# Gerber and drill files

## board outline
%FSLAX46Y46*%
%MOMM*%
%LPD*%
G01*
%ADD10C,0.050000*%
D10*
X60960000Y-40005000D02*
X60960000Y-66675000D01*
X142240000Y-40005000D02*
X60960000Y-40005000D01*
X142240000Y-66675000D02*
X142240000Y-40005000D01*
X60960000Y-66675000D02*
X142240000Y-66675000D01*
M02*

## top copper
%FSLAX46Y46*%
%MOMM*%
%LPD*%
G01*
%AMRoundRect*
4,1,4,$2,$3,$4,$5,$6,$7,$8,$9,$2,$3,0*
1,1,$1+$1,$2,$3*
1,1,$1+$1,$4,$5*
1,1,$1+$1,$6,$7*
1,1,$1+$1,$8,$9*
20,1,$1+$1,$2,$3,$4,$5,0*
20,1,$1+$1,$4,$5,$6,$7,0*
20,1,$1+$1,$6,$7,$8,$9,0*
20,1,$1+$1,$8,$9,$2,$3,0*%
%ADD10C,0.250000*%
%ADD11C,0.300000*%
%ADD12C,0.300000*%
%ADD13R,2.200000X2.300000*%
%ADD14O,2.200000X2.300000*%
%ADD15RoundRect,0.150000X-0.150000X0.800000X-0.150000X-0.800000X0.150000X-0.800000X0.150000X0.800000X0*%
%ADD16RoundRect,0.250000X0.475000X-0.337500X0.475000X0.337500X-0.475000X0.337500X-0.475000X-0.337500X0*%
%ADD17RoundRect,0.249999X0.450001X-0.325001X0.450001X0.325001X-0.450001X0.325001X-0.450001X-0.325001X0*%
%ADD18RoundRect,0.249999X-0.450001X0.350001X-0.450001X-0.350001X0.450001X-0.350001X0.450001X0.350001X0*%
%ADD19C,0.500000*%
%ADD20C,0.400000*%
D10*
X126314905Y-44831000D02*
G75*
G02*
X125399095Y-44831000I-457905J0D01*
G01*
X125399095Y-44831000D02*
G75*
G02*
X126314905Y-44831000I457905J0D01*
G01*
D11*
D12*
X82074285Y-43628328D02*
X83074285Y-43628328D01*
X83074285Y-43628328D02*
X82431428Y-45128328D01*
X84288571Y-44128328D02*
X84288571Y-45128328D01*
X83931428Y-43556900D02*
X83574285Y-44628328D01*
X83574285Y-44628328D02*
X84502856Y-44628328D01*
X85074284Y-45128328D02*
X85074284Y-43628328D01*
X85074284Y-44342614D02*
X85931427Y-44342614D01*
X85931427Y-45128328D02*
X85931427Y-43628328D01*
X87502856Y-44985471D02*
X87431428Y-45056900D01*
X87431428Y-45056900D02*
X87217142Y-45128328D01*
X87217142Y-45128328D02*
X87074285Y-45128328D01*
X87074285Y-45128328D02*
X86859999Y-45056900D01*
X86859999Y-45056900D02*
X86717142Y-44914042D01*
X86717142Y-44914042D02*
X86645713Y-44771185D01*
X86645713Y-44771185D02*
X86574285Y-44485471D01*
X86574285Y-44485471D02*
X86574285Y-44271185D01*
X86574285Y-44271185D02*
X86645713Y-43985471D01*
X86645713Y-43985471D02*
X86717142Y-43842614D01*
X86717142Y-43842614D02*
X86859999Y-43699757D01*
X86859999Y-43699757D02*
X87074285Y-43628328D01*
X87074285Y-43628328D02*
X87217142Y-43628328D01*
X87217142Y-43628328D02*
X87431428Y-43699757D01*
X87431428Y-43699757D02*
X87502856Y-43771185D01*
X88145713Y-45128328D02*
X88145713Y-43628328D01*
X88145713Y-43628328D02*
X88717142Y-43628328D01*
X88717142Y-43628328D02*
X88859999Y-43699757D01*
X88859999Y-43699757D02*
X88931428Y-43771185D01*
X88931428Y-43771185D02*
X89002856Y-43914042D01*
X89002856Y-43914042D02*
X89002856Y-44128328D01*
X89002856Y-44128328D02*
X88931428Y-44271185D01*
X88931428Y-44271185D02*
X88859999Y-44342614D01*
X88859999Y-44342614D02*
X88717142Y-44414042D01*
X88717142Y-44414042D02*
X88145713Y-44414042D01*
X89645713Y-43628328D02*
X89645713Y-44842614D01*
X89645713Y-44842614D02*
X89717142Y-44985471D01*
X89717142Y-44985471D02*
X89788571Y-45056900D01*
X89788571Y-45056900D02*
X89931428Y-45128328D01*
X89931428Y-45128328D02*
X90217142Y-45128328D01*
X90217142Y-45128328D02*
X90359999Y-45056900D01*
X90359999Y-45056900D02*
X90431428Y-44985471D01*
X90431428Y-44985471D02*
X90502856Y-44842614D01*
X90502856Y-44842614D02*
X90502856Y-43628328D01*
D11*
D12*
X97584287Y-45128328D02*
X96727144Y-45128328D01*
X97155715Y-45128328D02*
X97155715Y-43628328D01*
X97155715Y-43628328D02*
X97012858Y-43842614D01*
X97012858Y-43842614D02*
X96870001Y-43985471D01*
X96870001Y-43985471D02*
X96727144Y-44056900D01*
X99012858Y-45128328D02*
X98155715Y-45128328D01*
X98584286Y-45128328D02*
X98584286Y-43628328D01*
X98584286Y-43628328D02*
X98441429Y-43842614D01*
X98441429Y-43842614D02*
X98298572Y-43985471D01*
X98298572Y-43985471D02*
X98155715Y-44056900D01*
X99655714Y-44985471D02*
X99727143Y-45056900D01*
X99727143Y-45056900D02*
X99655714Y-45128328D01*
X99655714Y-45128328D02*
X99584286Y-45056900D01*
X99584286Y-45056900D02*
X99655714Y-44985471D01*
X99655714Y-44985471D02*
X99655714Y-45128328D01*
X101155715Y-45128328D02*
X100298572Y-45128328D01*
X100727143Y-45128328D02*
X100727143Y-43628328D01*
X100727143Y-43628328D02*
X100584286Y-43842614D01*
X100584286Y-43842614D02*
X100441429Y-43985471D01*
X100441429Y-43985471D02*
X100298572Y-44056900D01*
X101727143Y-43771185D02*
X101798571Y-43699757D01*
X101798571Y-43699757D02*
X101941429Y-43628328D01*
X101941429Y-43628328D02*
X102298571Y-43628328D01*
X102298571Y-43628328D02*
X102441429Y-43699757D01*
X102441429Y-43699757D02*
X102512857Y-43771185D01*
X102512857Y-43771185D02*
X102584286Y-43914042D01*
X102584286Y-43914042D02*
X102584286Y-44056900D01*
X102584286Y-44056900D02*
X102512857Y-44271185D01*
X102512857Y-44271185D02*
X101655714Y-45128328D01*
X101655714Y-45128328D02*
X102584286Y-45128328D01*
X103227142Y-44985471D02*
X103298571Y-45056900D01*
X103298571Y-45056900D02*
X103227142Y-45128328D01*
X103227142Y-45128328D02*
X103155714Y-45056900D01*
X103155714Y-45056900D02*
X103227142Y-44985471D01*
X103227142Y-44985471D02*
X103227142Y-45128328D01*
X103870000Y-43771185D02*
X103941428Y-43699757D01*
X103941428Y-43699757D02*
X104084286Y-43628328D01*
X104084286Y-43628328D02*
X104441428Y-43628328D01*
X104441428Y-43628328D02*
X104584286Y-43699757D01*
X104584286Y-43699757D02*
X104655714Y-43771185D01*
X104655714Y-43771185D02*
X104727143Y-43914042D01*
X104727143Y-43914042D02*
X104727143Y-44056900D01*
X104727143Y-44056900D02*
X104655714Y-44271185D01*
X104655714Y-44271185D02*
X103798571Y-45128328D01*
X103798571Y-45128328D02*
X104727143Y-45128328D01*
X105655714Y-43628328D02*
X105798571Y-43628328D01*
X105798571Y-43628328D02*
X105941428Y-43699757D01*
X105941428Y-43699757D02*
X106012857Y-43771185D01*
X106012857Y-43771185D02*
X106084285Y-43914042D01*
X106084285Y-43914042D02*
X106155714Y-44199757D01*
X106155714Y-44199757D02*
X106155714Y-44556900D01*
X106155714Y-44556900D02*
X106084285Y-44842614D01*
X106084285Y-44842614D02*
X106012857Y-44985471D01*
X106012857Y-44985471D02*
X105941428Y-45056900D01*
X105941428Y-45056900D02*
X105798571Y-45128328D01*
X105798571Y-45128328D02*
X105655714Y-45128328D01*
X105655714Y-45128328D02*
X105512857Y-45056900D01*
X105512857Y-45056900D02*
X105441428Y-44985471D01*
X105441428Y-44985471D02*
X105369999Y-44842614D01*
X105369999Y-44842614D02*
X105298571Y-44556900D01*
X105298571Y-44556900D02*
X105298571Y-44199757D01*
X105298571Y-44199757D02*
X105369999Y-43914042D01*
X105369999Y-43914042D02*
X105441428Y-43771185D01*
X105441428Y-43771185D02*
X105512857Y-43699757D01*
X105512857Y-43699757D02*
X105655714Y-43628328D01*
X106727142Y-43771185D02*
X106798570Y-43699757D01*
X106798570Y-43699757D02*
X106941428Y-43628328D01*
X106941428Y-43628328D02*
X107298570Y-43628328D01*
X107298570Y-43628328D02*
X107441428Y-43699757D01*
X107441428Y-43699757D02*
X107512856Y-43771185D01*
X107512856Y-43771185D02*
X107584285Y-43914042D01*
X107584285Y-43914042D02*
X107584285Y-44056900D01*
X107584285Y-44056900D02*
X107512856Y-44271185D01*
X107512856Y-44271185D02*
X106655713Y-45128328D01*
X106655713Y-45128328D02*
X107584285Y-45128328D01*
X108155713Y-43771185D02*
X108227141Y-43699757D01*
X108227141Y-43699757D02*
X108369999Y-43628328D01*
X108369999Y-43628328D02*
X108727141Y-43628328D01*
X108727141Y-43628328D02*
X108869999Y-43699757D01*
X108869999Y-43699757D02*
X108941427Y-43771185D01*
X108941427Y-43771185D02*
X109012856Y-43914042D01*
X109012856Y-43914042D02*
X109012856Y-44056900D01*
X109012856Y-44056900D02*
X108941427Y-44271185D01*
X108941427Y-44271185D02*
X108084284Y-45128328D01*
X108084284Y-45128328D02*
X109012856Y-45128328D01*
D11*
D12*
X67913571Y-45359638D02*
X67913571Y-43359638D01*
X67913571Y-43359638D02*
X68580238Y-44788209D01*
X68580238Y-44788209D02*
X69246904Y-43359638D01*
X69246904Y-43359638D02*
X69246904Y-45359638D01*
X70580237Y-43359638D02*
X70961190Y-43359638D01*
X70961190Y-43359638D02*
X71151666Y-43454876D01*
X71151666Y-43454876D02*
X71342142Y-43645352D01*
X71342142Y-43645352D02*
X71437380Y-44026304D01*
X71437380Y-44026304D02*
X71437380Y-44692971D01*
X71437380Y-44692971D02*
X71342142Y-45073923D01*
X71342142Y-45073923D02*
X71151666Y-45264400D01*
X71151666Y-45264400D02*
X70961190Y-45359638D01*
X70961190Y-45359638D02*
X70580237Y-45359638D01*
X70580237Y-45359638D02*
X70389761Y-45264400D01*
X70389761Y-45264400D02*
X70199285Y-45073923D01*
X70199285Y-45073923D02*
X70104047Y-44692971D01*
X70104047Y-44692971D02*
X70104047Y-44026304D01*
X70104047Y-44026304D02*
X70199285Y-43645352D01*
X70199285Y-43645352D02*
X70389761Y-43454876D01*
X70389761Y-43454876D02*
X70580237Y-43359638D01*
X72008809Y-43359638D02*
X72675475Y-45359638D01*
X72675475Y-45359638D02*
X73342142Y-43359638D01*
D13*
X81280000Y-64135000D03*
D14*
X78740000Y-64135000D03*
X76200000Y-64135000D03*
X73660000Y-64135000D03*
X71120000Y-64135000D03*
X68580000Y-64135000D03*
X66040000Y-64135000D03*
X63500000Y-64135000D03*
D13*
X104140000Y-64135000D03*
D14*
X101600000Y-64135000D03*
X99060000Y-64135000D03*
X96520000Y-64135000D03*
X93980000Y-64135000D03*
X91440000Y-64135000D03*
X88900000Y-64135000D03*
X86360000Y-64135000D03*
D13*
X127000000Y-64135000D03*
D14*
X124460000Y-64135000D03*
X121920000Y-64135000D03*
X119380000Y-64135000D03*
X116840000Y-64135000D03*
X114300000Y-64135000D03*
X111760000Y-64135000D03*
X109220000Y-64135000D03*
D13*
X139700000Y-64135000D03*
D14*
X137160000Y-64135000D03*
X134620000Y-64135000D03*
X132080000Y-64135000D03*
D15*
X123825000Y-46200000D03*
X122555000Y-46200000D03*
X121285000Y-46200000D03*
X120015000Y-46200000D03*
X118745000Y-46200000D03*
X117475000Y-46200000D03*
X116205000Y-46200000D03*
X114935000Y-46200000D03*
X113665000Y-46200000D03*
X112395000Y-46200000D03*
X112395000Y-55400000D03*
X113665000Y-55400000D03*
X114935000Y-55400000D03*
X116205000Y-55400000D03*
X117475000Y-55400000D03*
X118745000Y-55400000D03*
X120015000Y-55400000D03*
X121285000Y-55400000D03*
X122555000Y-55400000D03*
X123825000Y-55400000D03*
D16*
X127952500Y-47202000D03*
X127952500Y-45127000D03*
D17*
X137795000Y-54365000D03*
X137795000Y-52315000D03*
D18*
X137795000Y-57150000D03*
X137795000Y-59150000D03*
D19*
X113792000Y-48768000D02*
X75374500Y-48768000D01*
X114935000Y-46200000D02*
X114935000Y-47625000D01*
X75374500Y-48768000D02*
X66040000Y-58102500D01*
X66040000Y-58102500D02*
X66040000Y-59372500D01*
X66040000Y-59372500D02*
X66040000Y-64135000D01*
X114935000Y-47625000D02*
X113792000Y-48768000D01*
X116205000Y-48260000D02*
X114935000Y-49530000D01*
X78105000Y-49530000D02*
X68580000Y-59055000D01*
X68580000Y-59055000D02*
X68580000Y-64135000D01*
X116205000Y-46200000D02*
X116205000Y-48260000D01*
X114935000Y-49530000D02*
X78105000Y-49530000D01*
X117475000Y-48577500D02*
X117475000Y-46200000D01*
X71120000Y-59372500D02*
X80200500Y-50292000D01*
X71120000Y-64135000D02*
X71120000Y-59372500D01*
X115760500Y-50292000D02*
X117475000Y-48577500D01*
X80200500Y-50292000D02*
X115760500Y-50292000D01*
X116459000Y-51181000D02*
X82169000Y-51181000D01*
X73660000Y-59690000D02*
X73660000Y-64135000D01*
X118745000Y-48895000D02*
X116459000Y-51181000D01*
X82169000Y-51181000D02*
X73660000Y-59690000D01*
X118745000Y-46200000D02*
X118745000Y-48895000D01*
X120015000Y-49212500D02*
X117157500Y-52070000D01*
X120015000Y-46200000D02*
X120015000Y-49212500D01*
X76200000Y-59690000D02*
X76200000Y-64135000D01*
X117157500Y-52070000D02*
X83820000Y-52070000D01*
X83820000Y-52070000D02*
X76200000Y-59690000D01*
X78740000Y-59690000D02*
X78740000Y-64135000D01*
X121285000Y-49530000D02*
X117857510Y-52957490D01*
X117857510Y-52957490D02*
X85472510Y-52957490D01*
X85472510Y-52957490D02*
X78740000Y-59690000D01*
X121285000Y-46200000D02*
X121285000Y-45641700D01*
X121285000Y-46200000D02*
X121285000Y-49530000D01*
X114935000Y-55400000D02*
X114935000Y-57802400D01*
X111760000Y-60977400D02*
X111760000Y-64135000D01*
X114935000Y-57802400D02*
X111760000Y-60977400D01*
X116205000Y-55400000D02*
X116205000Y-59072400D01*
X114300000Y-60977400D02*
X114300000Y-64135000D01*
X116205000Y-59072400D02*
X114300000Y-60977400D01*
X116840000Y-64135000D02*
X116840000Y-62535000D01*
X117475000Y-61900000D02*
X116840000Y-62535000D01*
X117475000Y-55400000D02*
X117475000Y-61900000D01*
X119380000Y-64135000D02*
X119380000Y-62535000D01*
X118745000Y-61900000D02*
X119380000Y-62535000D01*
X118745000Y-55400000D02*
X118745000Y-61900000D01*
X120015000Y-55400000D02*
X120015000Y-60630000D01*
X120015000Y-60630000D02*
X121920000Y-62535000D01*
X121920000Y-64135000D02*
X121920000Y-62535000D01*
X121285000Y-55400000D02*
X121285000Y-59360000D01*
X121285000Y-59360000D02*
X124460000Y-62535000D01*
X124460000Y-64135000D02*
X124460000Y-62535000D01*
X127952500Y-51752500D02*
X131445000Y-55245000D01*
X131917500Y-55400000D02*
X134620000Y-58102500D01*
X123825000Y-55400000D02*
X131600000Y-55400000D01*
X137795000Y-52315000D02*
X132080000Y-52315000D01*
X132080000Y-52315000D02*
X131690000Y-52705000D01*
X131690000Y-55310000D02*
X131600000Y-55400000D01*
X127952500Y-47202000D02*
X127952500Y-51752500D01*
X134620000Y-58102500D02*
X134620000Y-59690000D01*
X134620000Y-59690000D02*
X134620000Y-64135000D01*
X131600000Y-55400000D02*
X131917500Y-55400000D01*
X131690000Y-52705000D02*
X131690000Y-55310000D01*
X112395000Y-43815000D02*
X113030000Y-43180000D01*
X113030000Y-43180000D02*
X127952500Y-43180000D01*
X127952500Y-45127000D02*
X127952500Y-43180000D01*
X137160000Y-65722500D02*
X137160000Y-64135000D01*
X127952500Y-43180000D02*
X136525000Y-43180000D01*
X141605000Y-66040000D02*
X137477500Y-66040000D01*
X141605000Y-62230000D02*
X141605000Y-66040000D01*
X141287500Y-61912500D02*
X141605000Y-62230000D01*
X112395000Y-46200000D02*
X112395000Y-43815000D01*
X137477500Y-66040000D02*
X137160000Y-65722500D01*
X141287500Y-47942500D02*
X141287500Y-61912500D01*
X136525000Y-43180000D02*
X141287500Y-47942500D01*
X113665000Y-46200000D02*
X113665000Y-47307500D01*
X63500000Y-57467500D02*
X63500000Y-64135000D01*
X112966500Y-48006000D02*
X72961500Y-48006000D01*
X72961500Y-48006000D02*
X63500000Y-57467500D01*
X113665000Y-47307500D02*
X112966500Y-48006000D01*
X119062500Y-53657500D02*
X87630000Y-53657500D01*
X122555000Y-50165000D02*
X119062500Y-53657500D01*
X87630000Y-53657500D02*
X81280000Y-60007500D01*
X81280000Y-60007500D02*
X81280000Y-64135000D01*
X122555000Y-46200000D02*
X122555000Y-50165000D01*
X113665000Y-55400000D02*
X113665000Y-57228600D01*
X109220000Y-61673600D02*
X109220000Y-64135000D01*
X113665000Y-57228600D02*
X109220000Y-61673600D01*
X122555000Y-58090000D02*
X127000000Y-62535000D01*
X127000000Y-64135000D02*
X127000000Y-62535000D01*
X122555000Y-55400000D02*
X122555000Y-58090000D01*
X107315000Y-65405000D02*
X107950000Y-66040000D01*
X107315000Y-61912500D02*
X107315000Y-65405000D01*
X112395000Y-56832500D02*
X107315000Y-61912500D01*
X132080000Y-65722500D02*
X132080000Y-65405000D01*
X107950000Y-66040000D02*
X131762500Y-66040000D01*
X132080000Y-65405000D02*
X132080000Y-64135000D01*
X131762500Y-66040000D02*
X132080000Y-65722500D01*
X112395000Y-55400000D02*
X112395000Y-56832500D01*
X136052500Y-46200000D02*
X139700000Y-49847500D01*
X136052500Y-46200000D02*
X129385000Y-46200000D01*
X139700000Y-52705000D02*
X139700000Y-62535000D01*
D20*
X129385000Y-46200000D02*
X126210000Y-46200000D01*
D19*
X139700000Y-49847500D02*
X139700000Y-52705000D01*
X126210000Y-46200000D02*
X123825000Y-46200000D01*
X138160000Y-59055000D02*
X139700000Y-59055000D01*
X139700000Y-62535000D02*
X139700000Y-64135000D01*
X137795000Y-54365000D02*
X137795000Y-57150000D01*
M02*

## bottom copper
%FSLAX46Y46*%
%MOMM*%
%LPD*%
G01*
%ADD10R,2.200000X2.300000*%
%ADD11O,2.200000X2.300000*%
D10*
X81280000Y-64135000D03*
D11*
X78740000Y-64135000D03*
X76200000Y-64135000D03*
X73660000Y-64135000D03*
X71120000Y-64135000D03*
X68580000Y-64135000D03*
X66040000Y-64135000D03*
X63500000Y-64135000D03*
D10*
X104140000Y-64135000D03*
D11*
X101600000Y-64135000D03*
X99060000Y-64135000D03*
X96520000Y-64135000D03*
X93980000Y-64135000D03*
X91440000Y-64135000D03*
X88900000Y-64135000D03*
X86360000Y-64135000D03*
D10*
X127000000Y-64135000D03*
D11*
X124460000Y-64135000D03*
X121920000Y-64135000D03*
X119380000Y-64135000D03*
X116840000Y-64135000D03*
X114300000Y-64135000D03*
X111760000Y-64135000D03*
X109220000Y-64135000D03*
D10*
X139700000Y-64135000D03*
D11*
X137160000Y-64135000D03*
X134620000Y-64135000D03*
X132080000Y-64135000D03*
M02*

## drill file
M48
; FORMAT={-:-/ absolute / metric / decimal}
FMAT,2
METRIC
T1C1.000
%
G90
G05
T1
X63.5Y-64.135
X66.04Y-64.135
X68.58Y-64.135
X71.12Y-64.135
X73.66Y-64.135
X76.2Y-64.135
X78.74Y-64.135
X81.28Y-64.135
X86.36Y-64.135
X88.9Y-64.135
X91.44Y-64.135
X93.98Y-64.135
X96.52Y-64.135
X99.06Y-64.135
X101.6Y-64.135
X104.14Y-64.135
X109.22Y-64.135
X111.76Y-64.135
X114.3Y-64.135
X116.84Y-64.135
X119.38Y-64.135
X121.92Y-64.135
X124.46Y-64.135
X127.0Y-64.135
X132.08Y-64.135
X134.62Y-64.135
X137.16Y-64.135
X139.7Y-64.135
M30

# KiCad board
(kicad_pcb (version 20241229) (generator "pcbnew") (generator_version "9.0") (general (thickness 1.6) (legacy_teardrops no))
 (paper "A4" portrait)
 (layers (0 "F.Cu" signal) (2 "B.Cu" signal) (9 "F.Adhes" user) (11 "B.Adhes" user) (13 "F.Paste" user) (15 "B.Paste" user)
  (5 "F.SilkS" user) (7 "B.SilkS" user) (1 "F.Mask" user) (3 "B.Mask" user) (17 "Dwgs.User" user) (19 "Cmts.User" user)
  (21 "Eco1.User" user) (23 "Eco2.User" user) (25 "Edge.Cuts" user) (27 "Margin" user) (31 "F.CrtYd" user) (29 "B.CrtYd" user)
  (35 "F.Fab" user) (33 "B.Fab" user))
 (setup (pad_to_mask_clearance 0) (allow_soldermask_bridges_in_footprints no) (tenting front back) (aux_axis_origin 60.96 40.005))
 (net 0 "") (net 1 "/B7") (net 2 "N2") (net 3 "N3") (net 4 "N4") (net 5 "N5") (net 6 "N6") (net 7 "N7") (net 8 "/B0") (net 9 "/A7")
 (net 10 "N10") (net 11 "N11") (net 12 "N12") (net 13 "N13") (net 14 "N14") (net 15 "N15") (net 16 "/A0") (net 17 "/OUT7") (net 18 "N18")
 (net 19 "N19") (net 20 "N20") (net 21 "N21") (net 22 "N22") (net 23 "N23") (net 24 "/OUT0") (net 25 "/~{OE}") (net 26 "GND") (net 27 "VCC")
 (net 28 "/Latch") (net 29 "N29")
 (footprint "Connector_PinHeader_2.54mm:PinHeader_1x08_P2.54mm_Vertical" (layer "F.Cu") (at 81.28 64.135 -90)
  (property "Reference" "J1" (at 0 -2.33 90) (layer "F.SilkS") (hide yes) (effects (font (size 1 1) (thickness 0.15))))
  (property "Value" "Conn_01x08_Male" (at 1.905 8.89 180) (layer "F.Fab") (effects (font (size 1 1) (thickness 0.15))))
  (pad "1" thru_hole rect (at 0 0 270) (size 2.3 2.2) (drill 1) (layers "*.Cu" "*.Mask") (remove_unused_layers no) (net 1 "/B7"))
  (pad "2" thru_hole oval (at 0 2.54 270) (size 2.3 2.2) (drill 1) (layers "*.Cu" "*.Mask") (remove_unused_layers no) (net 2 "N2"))
  (pad "3" thru_hole oval (at 0 5.08 270) (size 2.3 2.2) (drill 1) (layers "*.Cu" "*.Mask") (remove_unused_layers no) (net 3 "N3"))
  (pad "4" thru_hole oval (at 0 7.62 270) (size 2.3 2.2) (drill 1) (layers "*.Cu" "*.Mask") (remove_unused_layers no) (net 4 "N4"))
  (pad "5" thru_hole oval (at 0 10.16 270) (size 2.3 2.2) (drill 1) (layers "*.Cu" "*.Mask") (remove_unused_layers no) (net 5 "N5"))
  (pad "6" thru_hole oval (at 0 12.7 270) (size 2.3 2.2) (drill 1) (layers "*.Cu" "*.Mask") (remove_unused_layers no) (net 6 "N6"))
  (pad "7" thru_hole oval (at 0 15.24 270) (size 2.3 2.2) (drill 1) (layers "*.Cu" "*.Mask") (remove_unused_layers no) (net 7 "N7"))
  (pad "8" thru_hole oval (at 0 17.78 270) (size 2.3 2.2) (drill 1) (layers "*.Cu" "*.Mask") (remove_unused_layers no) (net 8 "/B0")))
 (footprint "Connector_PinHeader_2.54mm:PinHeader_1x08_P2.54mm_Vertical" (layer "F.Cu") (at 104.14 64.135 -90)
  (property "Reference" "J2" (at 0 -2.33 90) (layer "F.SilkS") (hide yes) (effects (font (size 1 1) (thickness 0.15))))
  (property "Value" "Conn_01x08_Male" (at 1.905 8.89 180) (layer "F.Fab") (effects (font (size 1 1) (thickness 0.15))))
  (pad "1" thru_hole rect (at 0 0 270) (size 2.3 2.2) (drill 1) (layers "*.Cu" "*.Mask") (remove_unused_layers no) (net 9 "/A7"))
  (pad "2" thru_hole oval (at 0 2.54 270) (size 2.3 2.2) (drill 1) (layers "*.Cu" "*.Mask") (remove_unused_layers no) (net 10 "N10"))
  (pad "3" thru_hole oval (at 0 5.08 270) (size 2.3 2.2) (drill 1) (layers "*.Cu" "*.Mask") (remove_unused_layers no) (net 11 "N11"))
  (pad "4" thru_hole oval (at 0 7.62 270) (size 2.3 2.2) (drill 1) (layers "*.Cu" "*.Mask") (remove_unused_layers no) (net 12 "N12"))
  (pad "5" thru_hole oval (at 0 10.16 270) (size 2.3 2.2) (drill 1) (layers "*.Cu" "*.Mask") (remove_unused_layers no) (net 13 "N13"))
  (pad "6" thru_hole oval (at 0 12.7 270) (size 2.3 2.2) (drill 1) (layers "*.Cu" "*.Mask") (remove_unused_layers no) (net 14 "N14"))
  (pad "7" thru_hole oval (at 0 15.24 270) (size 2.3 2.2) (drill 1) (layers "*.Cu" "*.Mask") (remove_unused_layers no) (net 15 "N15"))
  (pad "8" thru_hole oval (at 0 17.78 270) (size 2.3 2.2) (drill 1) (layers "*.Cu" "*.Mask") (remove_unused_layers no) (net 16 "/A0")))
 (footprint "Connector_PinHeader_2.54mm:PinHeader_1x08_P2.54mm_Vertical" (layer "F.Cu") (at 127 64.135 -90)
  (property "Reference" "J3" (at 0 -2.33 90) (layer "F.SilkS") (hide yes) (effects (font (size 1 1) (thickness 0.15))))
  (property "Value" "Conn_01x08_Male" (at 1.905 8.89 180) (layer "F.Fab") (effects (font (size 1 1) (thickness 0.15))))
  (pad "1" thru_hole rect (at 0 0 270) (size 2.3 2.2) (drill 1) (layers "*.Cu" "*.Mask") (remove_unused_layers no) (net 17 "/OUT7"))
  (pad "2" thru_hole oval (at 0 2.54 270) (size 2.3 2.2) (drill 1) (layers "*.Cu" "*.Mask") (remove_unused_layers no) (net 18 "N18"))
  (pad "3" thru_hole oval (at 0 5.08 270) (size 2.3 2.2) (drill 1) (layers "*.Cu" "*.Mask") (remove_unused_layers no) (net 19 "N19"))
  (pad "4" thru_hole oval (at 0 7.62 270) (size 2.3 2.2) (drill 1) (layers "*.Cu" "*.Mask") (remove_unused_layers no) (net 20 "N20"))
  (pad "5" thru_hole oval (at 0 10.16 270) (size 2.3 2.2) (drill 1) (layers "*.Cu" "*.Mask") (remove_unused_layers no) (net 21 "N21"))
  (pad "6" thru_hole oval (at 0 12.7 270) (size 2.3 2.2) (drill 1) (layers "*.Cu" "*.Mask") (remove_unused_layers no) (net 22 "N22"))
  (pad "7" thru_hole oval (at 0 15.24 270) (size 2.3 2.2) (drill 1) (layers "*.Cu" "*.Mask") (remove_unused_layers no) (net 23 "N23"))
  (pad "8" thru_hole oval (at 0 17.78 270) (size 2.3 2.2) (drill 1) (layers "*.Cu" "*.Mask") (remove_unused_layers no) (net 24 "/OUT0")))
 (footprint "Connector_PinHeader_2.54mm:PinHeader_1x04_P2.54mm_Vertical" (layer "F.Cu") (at 139.7 64.135 -90)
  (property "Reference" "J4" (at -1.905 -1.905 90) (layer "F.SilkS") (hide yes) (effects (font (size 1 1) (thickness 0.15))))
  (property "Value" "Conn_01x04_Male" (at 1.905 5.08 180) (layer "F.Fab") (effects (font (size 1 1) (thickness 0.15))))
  (pad "1" thru_hole rect (at 0 0 270) (size 2.3 2.2) (drill 1) (layers "*.Cu" "*.Mask") (remove_unused_layers no) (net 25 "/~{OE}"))
  (pad "2" thru_hole oval (at 0 2.54 270) (size 2.3 2.2) (drill 1) (layers "*.Cu" "*.Mask") (remove_unused_layers no) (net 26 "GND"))
  (pad "3" thru_hole oval (at 0 5.08 270) (size 2.3 2.2) (drill 1) (layers "*.Cu" "*.Mask") (remove_unused_layers no) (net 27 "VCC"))
  (pad "4" thru_hole oval (at 0 7.62 270) (size 2.3 2.2) (drill 1) (layers "*.Cu" "*.Mask") (remove_unused_layers no) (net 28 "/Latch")))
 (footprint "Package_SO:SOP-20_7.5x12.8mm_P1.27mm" (layer "F.Cu") (at 118.11 50.8 -90)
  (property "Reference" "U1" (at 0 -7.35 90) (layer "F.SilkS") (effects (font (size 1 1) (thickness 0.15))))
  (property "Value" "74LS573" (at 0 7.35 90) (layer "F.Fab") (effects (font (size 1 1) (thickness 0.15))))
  (pad "1" smd roundrect (at -4.6 -5.715 270) (size 1.9 0.6) (layers "F.Cu" "F.Mask" "F.Paste") (roundrect_rratio 0.25) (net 25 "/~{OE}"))
  (pad "2" smd roundrect (at -4.6 -4.445 270) (size 1.9 0.6) (layers "F.Cu" "F.Mask" "F.Paste") (roundrect_rratio 0.25) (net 1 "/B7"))
  (pad "3" smd roundrect (at -4.6 -3.175 270) (size 1.9 0.6) (layers "F.Cu" "F.Mask" "F.Paste") (roundrect_rratio 0.25) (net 2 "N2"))
  (pad "4" smd roundrect (at -4.6 -1.905 270) (size 1.9 0.6) (layers "F.Cu" "F.Mask" "F.Paste") (roundrect_rratio 0.25) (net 3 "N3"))
  (pad "5" smd roundrect (at -4.6 -0.635 270) (size 1.9 0.6) (layers "F.Cu" "F.Mask" "F.Paste") (roundrect_rratio 0.25) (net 4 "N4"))
  (pad "6" smd roundrect (at -4.6 0.635 270) (size 1.9 0.6) (layers "F.Cu" "F.Mask" "F.Paste") (roundrect_rratio 0.25) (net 5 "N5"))
  (pad "7" smd roundrect (at -4.6 1.905 270) (size 1.9 0.6) (layers "F.Cu" "F.Mask" "F.Paste") (roundrect_rratio 0.25) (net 6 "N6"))
  (pad "8" smd roundrect (at -4.6 3.175 270) (size 1.9 0.6) (layers "F.Cu" "F.Mask" "F.Paste") (roundrect_rratio 0.25) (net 7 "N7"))
  (pad "9" smd roundrect (at -4.6 4.445 270) (size 1.9 0.6) (layers "F.Cu" "F.Mask" "F.Paste") (roundrect_rratio 0.25) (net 8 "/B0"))
  (pad "10" smd roundrect (at -4.6 5.715 270) (size 1.9 0.6) (layers "F.Cu" "F.Mask" "F.Paste") (roundrect_rratio 0.25) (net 26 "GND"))
  (pad "11" smd roundrect (at 4.6 5.715 270) (size 1.9 0.6) (layers "F.Cu" "F.Mask" "F.Paste") (roundrect_rratio 0.25) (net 28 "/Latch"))
  (pad "12" smd roundrect (at 4.6 4.445 270) (size 1.9 0.6) (layers "F.Cu" "F.Mask" "F.Paste") (roundrect_rratio 0.25) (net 24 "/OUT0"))
  (pad "13" smd roundrect (at 4.6 3.175 270) (size 1.9 0.6) (layers "F.Cu" "F.Mask" "F.Paste") (roundrect_rratio 0.25) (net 23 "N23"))
  (pad "14" smd roundrect (at 4.6 1.905 270) (size 1.9 0.6) (layers "F.Cu" "F.Mask" "F.Paste") (roundrect_rratio 0.25) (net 22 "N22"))
  (pad "15" smd roundrect (at 4.6 0.635 270) (size 1.9 0.6) (layers "F.Cu" "F.Mask" "F.Paste") (roundrect_rratio 0.25) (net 21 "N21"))
  (pad "16" smd roundrect (at 4.6 -0.635 270) (size 1.9 0.6) (layers "F.Cu" "F.Mask" "F.Paste") (roundrect_rratio 0.25) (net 20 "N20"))
  (pad "17" smd roundrect (at 4.6 -1.905 270) (size 1.9 0.6) (layers "F.Cu" "F.Mask" "F.Paste") (roundrect_rratio 0.25) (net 19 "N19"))
  (pad "18" smd roundrect (at 4.6 -3.175 270) (size 1.9 0.6) (layers "F.Cu" "F.Mask" "F.Paste") (roundrect_rratio 0.25) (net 18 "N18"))
  (pad "19" smd roundrect (at 4.6 -4.445 270) (size 1.9 0.6) (layers "F.Cu" "F.Mask" "F.Paste") (roundrect_rratio 0.25) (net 17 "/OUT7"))
  (pad "20" smd roundrect (at 4.6 -5.715 270) (size 1.9 0.6) (layers "F.Cu" "F.Mask" "F.Paste") (roundrect_rratio 0.25) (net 27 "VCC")))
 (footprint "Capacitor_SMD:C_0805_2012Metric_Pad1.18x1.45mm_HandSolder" (layer "F.Cu") (at 127.9525 46.1645 90)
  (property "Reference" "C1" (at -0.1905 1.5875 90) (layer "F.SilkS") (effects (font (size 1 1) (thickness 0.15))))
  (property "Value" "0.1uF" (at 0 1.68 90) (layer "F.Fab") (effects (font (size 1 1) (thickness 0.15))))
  (pad "1" smd roundrect (at -1.0375 0 90) (size 1.175 1.45) (layers "F.Cu" "F.Mask" "F.Paste") (roundrect_rratio 0.2127659574)
   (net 27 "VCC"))
  (pad "2" smd roundrect (at 1.0375 0 90) (size 1.175 1.45) (layers "F.Cu" "F.Mask" "F.Paste") (roundrect_rratio 0.2127659574)
   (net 26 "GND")))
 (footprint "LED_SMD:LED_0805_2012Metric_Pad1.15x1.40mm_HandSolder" (layer "F.Cu") (at 137.795 53.34 90)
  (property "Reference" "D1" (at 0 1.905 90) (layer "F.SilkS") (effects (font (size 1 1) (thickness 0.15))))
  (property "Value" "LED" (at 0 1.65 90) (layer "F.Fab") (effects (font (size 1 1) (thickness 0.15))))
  (pad "1" smd roundrect (at -1.025 0 90) (size 1.15 1.4) (layers "F.Cu" "F.Mask" "F.Paste") (roundrect_rratio 0.2173904348) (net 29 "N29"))
  (pad "2" smd roundrect (at 1.025 0 90) (size 1.15 1.4) (layers "F.Cu" "F.Mask" "F.Paste") (roundrect_rratio 0.2173904348) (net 27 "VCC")))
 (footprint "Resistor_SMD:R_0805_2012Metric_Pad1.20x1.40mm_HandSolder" (layer "F.Cu") (at 137.795 58.15 -90)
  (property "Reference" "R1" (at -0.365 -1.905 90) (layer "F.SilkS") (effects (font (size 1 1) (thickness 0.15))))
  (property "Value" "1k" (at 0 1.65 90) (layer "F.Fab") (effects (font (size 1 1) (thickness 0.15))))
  (pad "1" smd roundrect (at -1 0 270) (size 1.2 1.4) (layers "F.Cu" "F.Mask" "F.Paste") (roundrect_rratio 0.2083325) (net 29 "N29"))
  (pad "2" smd roundrect (at 1 0 270) (size 1.2 1.4) (layers "F.Cu" "F.Mask" "F.Paste") (roundrect_rratio 0.2083325) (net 25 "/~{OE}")))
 (gr_circle (center 125.857 44.831) (end 126.314905 44.831) (stroke (width 0.25) (type solid)) (fill no) (layer "F.Cu"))
 (gr_line (start 60.96 40.005) (end 60.96 66.675) (stroke (width 0.05) (type solid)) (layer "Edge.Cuts"))
 (gr_line (start 142.24 40.005) (end 60.96 40.005) (stroke (width 0.05) (type solid)) (layer "Edge.Cuts"))
 (gr_line (start 142.24 66.675) (end 142.24 40.005) (stroke (width 0.05) (type solid)) (layer "Edge.Cuts"))
 (gr_line (start 60.96 66.675) (end 142.24 66.675) (stroke (width 0.05) (type solid)) (layer "Edge.Cuts"))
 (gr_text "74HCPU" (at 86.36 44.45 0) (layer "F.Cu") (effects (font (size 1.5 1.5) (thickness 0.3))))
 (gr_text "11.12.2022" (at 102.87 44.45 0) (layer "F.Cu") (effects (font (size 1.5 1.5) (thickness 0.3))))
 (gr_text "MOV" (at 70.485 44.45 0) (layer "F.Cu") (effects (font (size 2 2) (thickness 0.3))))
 (segment (start 113.792 48.768) (end 75.3745 48.768) (width 0.5) (layer "F.Cu") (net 7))
 (segment (start 114.935 46.2) (end 114.935 47.625) (width 0.5) (layer "F.Cu") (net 7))
 (segment (start 75.3745 48.768) (end 66.04 58.1025) (width 0.5) (layer "F.Cu") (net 7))
 (segment (start 66.04 58.1025) (end 66.04 59.3725) (width 0.5) (layer "F.Cu") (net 7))
 (segment (start 66.04 59.3725) (end 66.04 64.135) (width 0.5) (layer "F.Cu") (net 7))
 (segment (start 114.935 47.625) (end 113.792 48.768) (width 0.5) (layer "F.Cu") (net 7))
 (segment (start 116.205 48.26) (end 114.935 49.53) (width 0.5) (layer "F.Cu") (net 6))
 (segment (start 78.105 49.53) (end 68.58 59.055) (width 0.5) (layer "F.Cu") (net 6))
 (segment (start 68.58 59.055) (end 68.58 64.135) (width 0.5) (layer "F.Cu") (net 6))
 (segment (start 116.205 46.2) (end 116.205 48.26) (width 0.5) (layer "F.Cu") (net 6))
 (segment (start 114.935 49.53) (end 78.105 49.53) (width 0.5) (layer "F.Cu") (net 6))
 (segment (start 117.475 48.5775) (end 117.475 46.2) (width 0.5) (layer "F.Cu") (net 5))
 (segment (start 71.12 59.3725) (end 80.2005 50.292) (width 0.5) (layer "F.Cu") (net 5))
 (segment (start 71.12 64.135) (end 71.12 59.3725) (width 0.5) (layer "F.Cu") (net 5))
 (segment (start 115.7605 50.292) (end 117.475 48.5775) (width 0.5) (layer "F.Cu") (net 5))
 (segment (start 80.2005 50.292) (end 115.7605 50.292) (width 0.5) (layer "F.Cu") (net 5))
 (segment (start 116.459 51.181) (end 82.169 51.181) (width 0.5) (layer "F.Cu") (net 4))
 (segment (start 73.66 59.69) (end 73.66 64.135) (width 0.5) (layer "F.Cu") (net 4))
 (segment (start 118.745 48.895) (end 116.459 51.181) (width 0.5) (layer "F.Cu") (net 4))
 (segment (start 82.169 51.181) (end 73.66 59.69) (width 0.5) (layer "F.Cu") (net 4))
 (segment (start 118.745 46.2) (end 118.745 48.895) (width 0.5) (layer "F.Cu") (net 4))
 (segment (start 120.015 49.2125) (end 117.1575 52.07) (width 0.5) (layer "F.Cu") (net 3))
 (segment (start 120.015 46.2) (end 120.015 49.2125) (width 0.5) (layer "F.Cu") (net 3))
 (segment (start 76.2 59.69) (end 76.2 64.135) (width 0.5) (layer "F.Cu") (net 3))
 (segment (start 117.1575 52.07) (end 83.82 52.07) (width 0.5) (layer "F.Cu") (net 3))
 (segment (start 83.82 52.07) (end 76.2 59.69) (width 0.5) (layer "F.Cu") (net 3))
 (segment (start 78.74 59.69) (end 78.74 64.135) (width 0.5) (layer "F.Cu") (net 2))
 (segment (start 121.285 49.53) (end 117.85751 52.95749) (width 0.5) (layer "F.Cu") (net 2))
 (segment (start 117.85751 52.95749) (end 85.47251 52.95749) (width 0.5) (layer "F.Cu") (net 2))
 (segment (start 85.47251 52.95749) (end 78.74 59.69) (width 0.5) (layer "F.Cu") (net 2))
 (segment (start 121.285 46.2) (end 121.285 45.6417) (width 0.5) (layer "F.Cu") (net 2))
 (segment (start 121.285 46.2) (end 121.285 49.53) (width 0.5) (layer "F.Cu") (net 2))
 (segment (start 114.935 55.4) (end 114.935 57.8024) (width 0.5) (layer "F.Cu") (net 23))
 (segment (start 111.76 60.9774) (end 111.76 64.135) (width 0.5) (layer "F.Cu") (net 23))
 (segment (start 114.935 57.8024) (end 111.76 60.9774) (width 0.5) (layer "F.Cu") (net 23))
 (segment (start 116.205 55.4) (end 116.205 59.0724) (width 0.5) (layer "F.Cu") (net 22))
 (segment (start 114.3 60.9774) (end 114.3 64.135) (width 0.5) (layer "F.Cu") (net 22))
 (segment (start 116.205 59.0724) (end 114.3 60.9774) (width 0.5) (layer "F.Cu") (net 22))
 (segment (start 116.84 64.135) (end 116.84 62.535) (width 0.5) (layer "F.Cu") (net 21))
 (segment (start 117.475 61.9) (end 116.84 62.535) (width 0.5) (layer "F.Cu") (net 21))
 (segment (start 117.475 55.4) (end 117.475 61.9) (width 0.5) (layer "F.Cu") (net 21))
 (segment (start 119.38 64.135) (end 119.38 62.535) (width 0.5) (layer "F.Cu") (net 20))
 (segment (start 118.745 61.9) (end 119.38 62.535) (width 0.5) (layer "F.Cu") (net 20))
 (segment (start 118.745 55.4) (end 118.745 61.9) (width 0.5) (layer "F.Cu") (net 20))
 (segment (start 120.015 55.4) (end 120.015 60.63) (width 0.5) (layer "F.Cu") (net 19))
 (segment (start 120.015 60.63) (end 121.92 62.535) (width 0.5) (layer "F.Cu") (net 19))
 (segment (start 121.92 64.135) (end 121.92 62.535) (width 0.5) (layer "F.Cu") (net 19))
 (segment (start 121.285 55.4) (end 121.285 59.36) (width 0.5) (layer "F.Cu") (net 18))
 (segment (start 121.285 59.36) (end 124.46 62.535) (width 0.5) (layer "F.Cu") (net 18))
 (segment (start 124.46 64.135) (end 124.46 62.535) (width 0.5) (layer "F.Cu") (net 18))
 (segment (start 127.9525 51.7525) (end 131.445 55.245) (width 0.5) (layer "F.Cu") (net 27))
 (segment (start 131.9175 55.4) (end 134.62 58.1025) (width 0.5) (layer "F.Cu") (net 27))
 (segment (start 123.825 55.4) (end 131.6 55.4) (width 0.5) (layer "F.Cu") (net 27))
 (segment (start 137.795 52.315) (end 132.08 52.315) (width 0.5) (layer "F.Cu") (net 27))
 (segment (start 132.08 52.315) (end 131.69 52.705) (width 0.5) (layer "F.Cu") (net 27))
 (segment (start 131.69 55.31) (end 131.6 55.4) (width 0.5) (layer "F.Cu") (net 27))
 (segment (start 127.9525 47.202) (end 127.9525 51.7525) (width 0.5) (layer "F.Cu") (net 27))
 (segment (start 134.62 58.1025) (end 134.62 59.69) (width 0.5) (layer "F.Cu") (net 27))
 (segment (start 134.62 59.69) (end 134.62 64.135) (width 0.5) (layer "F.Cu") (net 27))
 (segment (start 131.6 55.4) (end 131.9175 55.4) (width 0.5) (layer "F.Cu") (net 27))
 (segment (start 131.69 52.705) (end 131.69 55.31) (width 0.5) (layer "F.Cu") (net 27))
 (segment (start 112.395 43.815) (end 113.03 43.18) (width 0.5) (layer "F.Cu") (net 26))
 (segment (start 113.03 43.18) (end 127.9525 43.18) (width 0.5) (layer "F.Cu") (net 26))
 (segment (start 127.9525 45.127) (end 127.9525 43.18) (width 0.5) (layer "F.Cu") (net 26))
 (segment (start 137.16 65.7225) (end 137.16 64.135) (width 0.5) (layer "F.Cu") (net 26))
 (segment (start 127.9525 43.18) (end 136.525 43.18) (width 0.5) (layer "F.Cu") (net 26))
 (segment (start 141.605 66.04) (end 137.4775 66.04) (width 0.5) (layer "F.Cu") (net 26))
 (segment (start 141.605 62.23) (end 141.605 66.04) (width 0.5) (layer "F.Cu") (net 26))
 (segment (start 141.2875 61.9125) (end 141.605 62.23) (width 0.5) (layer "F.Cu") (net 26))
 (segment (start 112.395 46.2) (end 112.395 43.815) (width 0.5) (layer "F.Cu") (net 26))
 (segment (start 137.4775 66.04) (end 137.16 65.7225) (width 0.5) (layer "F.Cu") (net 26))
 (segment (start 141.2875 47.9425) (end 141.2875 61.9125) (width 0.5) (layer "F.Cu") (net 26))
 (segment (start 136.525 43.18) (end 141.2875 47.9425) (width 0.5) (layer "F.Cu") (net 26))
 (segment (start 113.665 46.2) (end 113.665 47.3075) (width 0.5) (layer "F.Cu") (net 8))
 (segment (start 63.5 57.4675) (end 63.5 64.135) (width 0.5) (layer "F.Cu") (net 8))
 (segment (start 112.9665 48.006) (end 72.9615 48.006) (width 0.5) (layer "F.Cu") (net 8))
 (segment (start 72.9615 48.006) (end 63.5 57.4675) (width 0.5) (layer "F.Cu") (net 8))
 (segment (start 113.665 47.3075) (end 112.9665 48.006) (width 0.5) (layer "F.Cu") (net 8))
 (segment (start 119.0625 53.6575) (end 87.63 53.6575) (width 0.5) (layer "F.Cu") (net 1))
 (segment (start 122.555 50.165) (end 119.0625 53.6575) (width 0.5) (layer "F.Cu") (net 1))
 (segment (start 87.63 53.6575) (end 81.28 60.0075) (width 0.5) (layer "F.Cu") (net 1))
 (segment (start 81.28 60.0075) (end 81.28 64.135) (width 0.5) (layer "F.Cu") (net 1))
 (segment (start 122.555 46.2) (end 122.555 50.165) (width 0.5) (layer "F.Cu") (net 1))
 (segment (start 113.665 55.4) (end 113.665 57.2286) (width 0.5) (layer "F.Cu") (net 24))
 (segment (start 109.22 61.6736) (end 109.22 64.135) (width 0.5) (layer "F.Cu") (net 24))
 (segment (start 113.665 57.2286) (end 109.22 61.6736) (width 0.5) (layer "F.Cu") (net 24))
 (segment (start 122.555 58.09) (end 127 62.535) (width 0.5) (layer "F.Cu") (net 17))
 (segment (start 127 64.135) (end 127 62.535) (width 0.5) (layer "F.Cu") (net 17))
 (segment (start 122.555 55.4) (end 122.555 58.09) (width 0.5) (layer "F.Cu") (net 17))
 (segment (start 107.315 65.405) (end 107.95 66.04) (width 0.5) (layer "F.Cu") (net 28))
 (segment (start 107.315 61.9125) (end 107.315 65.405) (width 0.5) (layer "F.Cu") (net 28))
 (segment (start 112.395 56.8325) (end 107.315 61.9125) (width 0.5) (layer "F.Cu") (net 28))
 (segment (start 132.08 65.7225) (end 132.08 65.405) (width 0.5) (layer "F.Cu") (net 28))
 (segment (start 107.95 66.04) (end 131.7625 66.04) (width 0.5) (layer "F.Cu") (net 28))
 (segment (start 132.08 65.405) (end 132.08 64.135) (width 0.5) (layer "F.Cu") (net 28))
 (segment (start 131.7625 66.04) (end 132.08 65.7225) (width 0.5) (layer "F.Cu") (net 28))
 (segment (start 112.395 55.4) (end 112.395 56.8325) (width 0.5) (layer "F.Cu") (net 28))
 (segment (start 136.0525 46.2) (end 139.7 49.8475) (width 0.5) (layer "F.Cu") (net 25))
 (segment (start 136.0525 46.2) (end 129.385 46.2) (width 0.5) (layer "F.Cu") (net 25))
 (segment (start 139.7 52.705) (end 139.7 62.535) (width 0.5) (layer "F.Cu") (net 25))
 (segment (start 129.385 46.2) (end 126.21 46.2) (width 0.4) (layer "F.Cu") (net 25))
 (segment (start 139.7 49.8475) (end 139.7 52.705) (width 0.5) (layer "F.Cu") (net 25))
 (segment (start 126.21 46.2) (end 123.825 46.2) (width 0.5) (layer "F.Cu") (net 25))
 (segment (start 138.16 59.055) (end 139.7 59.055) (width 0.5) (layer "F.Cu") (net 25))
 (segment (start 139.7 62.535) (end 139.7 64.135) (width 0.5) (layer "F.Cu") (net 25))
 (segment (start 137.795 54.365) (end 137.795 57.15) (width 0.5) (layer "F.Cu") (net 29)))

